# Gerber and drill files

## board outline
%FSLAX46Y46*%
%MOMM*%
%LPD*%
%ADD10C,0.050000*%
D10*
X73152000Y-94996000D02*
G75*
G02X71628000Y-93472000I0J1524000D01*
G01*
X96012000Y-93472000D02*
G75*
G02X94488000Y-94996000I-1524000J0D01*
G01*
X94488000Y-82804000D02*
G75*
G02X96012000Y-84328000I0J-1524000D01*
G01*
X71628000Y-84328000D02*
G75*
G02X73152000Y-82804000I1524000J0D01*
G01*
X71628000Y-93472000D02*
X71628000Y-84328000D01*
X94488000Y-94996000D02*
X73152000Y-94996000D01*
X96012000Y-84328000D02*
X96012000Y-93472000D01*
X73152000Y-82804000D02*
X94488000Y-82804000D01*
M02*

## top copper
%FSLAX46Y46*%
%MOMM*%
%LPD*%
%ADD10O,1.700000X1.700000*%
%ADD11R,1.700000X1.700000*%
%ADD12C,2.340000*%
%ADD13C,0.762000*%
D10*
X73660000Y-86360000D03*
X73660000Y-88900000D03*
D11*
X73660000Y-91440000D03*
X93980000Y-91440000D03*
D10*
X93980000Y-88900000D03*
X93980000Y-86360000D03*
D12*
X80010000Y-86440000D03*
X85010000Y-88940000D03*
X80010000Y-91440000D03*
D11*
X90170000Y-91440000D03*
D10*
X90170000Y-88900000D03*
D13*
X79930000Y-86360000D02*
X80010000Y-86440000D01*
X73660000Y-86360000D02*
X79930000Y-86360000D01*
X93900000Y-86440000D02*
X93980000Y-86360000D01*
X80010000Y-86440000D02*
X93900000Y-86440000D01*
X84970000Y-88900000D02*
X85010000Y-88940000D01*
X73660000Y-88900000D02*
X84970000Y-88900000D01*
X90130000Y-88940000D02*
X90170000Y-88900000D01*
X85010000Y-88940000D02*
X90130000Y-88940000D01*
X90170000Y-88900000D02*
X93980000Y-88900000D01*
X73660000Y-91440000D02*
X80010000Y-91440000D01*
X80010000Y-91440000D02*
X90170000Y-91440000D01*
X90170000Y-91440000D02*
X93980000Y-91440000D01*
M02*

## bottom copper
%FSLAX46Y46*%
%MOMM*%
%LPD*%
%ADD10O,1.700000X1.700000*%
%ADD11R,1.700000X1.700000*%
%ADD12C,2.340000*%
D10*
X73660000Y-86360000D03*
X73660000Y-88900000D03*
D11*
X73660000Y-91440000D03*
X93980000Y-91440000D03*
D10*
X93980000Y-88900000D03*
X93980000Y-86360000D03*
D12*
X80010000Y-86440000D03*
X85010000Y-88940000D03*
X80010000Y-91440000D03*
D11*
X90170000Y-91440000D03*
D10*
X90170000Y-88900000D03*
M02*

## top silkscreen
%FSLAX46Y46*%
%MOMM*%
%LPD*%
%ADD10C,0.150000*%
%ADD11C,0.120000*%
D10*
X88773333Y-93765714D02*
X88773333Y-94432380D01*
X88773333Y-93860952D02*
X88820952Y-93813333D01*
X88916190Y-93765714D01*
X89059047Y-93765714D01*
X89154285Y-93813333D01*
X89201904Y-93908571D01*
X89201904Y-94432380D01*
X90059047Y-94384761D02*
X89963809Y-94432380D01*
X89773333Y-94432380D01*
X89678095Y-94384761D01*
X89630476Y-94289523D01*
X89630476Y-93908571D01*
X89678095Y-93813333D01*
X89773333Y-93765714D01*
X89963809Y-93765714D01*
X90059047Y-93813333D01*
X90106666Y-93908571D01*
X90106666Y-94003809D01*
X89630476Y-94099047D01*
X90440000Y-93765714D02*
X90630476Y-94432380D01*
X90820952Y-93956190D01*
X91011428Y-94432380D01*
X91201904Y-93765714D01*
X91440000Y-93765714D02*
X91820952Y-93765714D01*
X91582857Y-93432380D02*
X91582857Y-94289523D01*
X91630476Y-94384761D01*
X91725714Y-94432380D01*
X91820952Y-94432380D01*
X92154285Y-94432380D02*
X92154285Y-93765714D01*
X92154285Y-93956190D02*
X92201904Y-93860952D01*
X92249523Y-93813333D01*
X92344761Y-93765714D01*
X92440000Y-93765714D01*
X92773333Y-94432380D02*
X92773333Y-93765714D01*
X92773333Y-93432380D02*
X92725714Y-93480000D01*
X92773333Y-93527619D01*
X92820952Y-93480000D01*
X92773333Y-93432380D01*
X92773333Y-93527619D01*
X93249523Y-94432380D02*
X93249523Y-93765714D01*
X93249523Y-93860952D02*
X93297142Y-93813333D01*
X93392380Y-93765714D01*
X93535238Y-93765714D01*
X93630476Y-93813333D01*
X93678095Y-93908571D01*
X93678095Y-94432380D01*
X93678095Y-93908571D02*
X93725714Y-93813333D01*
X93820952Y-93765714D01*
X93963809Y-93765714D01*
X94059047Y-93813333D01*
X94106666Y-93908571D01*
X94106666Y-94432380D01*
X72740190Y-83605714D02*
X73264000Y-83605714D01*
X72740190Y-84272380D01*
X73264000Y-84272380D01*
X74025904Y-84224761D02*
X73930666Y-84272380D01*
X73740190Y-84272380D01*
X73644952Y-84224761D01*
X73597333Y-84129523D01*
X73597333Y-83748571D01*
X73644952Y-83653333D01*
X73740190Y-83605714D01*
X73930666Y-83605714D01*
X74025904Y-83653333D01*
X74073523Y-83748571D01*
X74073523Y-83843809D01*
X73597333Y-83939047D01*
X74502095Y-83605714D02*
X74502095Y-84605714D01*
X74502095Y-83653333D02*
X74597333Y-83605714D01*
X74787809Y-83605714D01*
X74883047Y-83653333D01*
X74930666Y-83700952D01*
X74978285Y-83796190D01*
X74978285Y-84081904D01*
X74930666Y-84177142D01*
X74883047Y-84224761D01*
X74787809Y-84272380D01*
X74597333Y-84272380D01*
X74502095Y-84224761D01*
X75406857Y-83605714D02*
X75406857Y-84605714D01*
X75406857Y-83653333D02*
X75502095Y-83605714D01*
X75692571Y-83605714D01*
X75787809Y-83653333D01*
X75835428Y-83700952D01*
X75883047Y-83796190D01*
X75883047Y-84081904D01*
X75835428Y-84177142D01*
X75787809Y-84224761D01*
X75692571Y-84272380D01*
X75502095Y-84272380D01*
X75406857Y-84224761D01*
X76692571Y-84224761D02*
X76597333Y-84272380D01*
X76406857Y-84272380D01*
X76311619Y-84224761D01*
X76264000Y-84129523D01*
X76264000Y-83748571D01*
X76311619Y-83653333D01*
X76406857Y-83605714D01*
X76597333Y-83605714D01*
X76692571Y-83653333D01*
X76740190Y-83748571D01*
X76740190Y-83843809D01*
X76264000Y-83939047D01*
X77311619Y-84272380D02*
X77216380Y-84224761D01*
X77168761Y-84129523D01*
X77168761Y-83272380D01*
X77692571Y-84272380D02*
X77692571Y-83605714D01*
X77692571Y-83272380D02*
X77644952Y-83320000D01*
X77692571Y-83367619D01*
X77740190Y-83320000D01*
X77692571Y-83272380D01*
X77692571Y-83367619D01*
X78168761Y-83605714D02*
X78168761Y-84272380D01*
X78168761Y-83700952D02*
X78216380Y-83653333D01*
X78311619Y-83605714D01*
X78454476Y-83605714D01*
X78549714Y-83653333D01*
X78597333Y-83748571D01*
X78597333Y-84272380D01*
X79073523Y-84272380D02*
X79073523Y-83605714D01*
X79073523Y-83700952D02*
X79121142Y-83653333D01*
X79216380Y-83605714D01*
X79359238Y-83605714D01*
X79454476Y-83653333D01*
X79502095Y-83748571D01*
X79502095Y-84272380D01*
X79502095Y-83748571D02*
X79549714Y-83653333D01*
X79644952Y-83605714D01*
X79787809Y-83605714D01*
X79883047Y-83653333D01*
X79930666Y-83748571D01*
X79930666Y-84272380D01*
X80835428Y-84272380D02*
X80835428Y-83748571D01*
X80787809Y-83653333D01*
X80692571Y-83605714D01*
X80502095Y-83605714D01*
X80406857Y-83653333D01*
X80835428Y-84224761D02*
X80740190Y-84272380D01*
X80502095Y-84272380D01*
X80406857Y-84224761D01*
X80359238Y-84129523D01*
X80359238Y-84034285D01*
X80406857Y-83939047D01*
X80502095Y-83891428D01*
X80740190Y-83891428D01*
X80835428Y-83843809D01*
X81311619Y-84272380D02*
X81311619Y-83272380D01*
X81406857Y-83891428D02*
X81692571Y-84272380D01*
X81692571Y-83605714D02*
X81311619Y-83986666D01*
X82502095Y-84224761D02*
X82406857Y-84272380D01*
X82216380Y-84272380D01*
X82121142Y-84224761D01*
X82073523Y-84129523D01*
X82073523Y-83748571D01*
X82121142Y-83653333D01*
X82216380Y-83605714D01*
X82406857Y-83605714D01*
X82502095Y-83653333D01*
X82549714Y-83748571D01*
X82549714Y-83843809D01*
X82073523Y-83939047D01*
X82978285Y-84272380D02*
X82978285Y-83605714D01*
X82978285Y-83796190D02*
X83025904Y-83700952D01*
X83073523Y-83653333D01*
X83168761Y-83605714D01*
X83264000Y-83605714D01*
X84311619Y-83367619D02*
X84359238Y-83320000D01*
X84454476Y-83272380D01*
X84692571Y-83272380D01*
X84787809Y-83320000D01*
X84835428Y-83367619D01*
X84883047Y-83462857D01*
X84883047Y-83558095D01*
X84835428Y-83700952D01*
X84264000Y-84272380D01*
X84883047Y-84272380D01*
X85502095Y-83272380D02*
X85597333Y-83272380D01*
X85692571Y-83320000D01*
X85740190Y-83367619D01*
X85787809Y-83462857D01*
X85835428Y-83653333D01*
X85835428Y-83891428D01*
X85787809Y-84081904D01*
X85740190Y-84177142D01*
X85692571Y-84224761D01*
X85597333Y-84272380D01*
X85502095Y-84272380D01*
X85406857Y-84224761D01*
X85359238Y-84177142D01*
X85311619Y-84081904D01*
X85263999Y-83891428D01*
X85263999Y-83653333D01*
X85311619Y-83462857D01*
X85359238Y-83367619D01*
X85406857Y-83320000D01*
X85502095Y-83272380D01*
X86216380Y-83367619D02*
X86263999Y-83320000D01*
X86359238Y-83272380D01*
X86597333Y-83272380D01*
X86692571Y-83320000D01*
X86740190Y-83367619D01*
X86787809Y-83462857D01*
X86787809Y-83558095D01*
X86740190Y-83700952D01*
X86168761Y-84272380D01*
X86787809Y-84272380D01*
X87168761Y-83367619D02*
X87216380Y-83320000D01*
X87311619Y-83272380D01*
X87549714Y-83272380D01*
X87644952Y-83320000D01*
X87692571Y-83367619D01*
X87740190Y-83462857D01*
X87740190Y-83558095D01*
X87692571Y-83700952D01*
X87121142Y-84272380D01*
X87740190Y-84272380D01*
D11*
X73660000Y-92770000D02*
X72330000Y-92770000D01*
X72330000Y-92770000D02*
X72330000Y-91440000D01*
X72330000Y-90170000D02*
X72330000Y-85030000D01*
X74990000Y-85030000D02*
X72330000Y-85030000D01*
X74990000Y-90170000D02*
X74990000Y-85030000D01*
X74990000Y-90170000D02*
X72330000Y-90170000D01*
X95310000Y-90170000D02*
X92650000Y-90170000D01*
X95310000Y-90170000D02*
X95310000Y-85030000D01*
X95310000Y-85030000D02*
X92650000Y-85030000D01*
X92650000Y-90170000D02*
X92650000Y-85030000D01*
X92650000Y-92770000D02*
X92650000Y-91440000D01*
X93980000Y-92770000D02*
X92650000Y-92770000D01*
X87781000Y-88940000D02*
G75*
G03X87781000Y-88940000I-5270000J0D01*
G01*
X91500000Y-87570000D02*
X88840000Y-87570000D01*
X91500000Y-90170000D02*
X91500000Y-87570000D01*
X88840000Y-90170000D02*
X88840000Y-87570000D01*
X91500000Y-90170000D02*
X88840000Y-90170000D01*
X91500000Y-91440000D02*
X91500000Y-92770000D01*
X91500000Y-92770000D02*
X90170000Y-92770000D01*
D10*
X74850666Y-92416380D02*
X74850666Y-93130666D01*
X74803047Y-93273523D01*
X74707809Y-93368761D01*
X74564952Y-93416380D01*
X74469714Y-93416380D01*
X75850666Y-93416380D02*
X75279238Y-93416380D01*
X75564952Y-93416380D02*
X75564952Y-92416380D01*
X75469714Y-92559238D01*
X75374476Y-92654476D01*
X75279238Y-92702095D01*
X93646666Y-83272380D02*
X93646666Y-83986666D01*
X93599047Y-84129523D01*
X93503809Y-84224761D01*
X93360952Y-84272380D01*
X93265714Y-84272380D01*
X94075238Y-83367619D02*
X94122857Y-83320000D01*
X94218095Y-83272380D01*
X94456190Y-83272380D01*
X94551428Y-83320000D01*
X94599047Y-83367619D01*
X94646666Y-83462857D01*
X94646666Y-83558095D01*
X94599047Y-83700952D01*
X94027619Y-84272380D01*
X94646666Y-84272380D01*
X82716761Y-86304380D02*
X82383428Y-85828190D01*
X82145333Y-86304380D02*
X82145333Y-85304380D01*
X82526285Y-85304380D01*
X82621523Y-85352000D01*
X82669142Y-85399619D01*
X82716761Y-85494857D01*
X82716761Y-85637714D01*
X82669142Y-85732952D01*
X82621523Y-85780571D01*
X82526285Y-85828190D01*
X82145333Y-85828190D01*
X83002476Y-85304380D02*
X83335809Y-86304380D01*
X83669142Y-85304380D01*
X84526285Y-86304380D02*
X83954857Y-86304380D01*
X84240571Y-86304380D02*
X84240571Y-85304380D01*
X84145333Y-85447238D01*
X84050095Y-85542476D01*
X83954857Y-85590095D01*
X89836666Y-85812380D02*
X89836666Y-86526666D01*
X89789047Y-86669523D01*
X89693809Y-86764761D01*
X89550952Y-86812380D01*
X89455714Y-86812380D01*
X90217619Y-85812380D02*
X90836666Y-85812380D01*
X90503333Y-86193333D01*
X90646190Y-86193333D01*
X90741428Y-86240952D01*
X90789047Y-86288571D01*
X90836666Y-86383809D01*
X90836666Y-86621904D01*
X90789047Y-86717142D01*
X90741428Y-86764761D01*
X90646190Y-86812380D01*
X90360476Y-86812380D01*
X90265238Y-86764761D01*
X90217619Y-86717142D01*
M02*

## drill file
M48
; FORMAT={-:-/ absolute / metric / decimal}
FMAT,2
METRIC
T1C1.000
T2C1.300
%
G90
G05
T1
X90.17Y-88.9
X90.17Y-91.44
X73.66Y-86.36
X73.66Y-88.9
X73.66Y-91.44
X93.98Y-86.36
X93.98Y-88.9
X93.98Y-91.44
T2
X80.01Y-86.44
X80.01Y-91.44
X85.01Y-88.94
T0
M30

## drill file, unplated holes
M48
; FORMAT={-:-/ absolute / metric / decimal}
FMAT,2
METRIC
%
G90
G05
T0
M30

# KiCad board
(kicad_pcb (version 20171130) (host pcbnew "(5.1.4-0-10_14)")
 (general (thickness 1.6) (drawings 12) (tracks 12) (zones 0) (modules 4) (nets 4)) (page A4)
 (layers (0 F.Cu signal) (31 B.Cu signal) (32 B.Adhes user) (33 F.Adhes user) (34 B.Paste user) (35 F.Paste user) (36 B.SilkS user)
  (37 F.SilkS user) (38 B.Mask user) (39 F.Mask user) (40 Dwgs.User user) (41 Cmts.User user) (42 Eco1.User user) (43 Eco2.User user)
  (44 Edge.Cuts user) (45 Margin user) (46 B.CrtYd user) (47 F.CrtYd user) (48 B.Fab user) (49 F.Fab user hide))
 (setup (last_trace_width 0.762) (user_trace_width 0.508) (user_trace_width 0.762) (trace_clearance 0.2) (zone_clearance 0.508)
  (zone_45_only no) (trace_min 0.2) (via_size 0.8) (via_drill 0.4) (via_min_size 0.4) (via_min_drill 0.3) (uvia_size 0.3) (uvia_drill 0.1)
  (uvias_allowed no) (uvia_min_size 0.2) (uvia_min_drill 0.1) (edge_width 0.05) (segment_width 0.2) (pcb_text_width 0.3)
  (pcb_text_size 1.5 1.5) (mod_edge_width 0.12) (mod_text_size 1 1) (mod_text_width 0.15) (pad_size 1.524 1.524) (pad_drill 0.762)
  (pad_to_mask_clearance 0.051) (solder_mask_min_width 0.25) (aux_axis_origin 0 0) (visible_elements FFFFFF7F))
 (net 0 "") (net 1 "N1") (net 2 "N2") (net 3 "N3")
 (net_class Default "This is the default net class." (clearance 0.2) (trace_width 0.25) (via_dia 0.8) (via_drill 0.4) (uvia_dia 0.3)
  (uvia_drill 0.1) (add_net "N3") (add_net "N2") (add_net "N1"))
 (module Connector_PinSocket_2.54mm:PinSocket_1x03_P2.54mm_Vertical (layer F.Cu) (at 73.66 91.44 180)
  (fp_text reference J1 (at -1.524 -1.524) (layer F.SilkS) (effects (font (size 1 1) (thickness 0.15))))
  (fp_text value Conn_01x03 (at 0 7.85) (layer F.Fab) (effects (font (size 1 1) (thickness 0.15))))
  (fp_line (start 0 -1.33) (end 1.33 -1.33) (layer F.SilkS) (width 0.12))
  (fp_line (start 1.33 -1.33) (end 1.33 0) (layer F.SilkS) (width 0.12))
  (fp_line (start 1.33 1.27) (end 1.33 6.41) (layer F.SilkS) (width 0.12))
  (fp_line (start -1.33 6.41) (end 1.33 6.41) (layer F.SilkS) (width 0.12))
  (fp_line (start -1.33 1.27) (end -1.33 6.41) (layer F.SilkS) (width 0.12))
  (fp_line (start -1.33 1.27) (end 1.33 1.27) (layer F.SilkS) (width 0.12))
  (pad 3 thru_hole oval (at 0 5.08 180) (size 1.7 1.7) (drill 1) (layers *.Cu *.Mask) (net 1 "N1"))
  (pad 2 thru_hole oval (at 0 2.54 180) (size 1.7 1.7) (drill 1) (layers *.Cu *.Mask) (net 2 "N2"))
  (pad 1 thru_hole rect (at 0 0 180) (size 1.7 1.7) (drill 1) (layers *.Cu *.Mask) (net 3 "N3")))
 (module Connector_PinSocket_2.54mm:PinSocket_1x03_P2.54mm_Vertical (layer F.Cu) (at 93.98 91.44 180)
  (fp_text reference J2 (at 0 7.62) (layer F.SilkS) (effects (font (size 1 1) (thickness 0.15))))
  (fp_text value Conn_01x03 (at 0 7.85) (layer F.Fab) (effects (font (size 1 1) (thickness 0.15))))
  (fp_line (start -1.33 1.27) (end 1.33 1.27) (layer F.SilkS) (width 0.12))
  (fp_line (start -1.33 1.27) (end -1.33 6.41) (layer F.SilkS) (width 0.12))
  (fp_line (start -1.33 6.41) (end 1.33 6.41) (layer F.SilkS) (width 0.12))
  (fp_line (start 1.33 1.27) (end 1.33 6.41) (layer F.SilkS) (width 0.12))
  (fp_line (start 1.33 -1.33) (end 1.33 0) (layer F.SilkS) (width 0.12))
  (fp_line (start 0 -1.33) (end 1.33 -1.33) (layer F.SilkS) (width 0.12))
  (pad 1 thru_hole rect (at 0 0 180) (size 1.7 1.7) (drill 1) (layers *.Cu *.Mask) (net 3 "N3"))
  (pad 2 thru_hole oval (at 0 2.54 180) (size 1.7 1.7) (drill 1) (layers *.Cu *.Mask) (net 2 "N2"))
  (pad 3 thru_hole oval (at 0 5.08 180) (size 1.7 1.7) (drill 1) (layers *.Cu *.Mask) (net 1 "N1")))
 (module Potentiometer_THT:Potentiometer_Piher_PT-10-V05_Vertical (layer F.Cu) (at 80.01 91.44)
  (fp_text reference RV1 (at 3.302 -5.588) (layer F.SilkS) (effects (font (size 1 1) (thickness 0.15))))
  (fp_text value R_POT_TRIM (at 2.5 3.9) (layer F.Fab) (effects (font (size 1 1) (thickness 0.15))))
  (fp_circle (center 2.501 -2.5) (end 7.771 -2.5) (layer F.SilkS) (width 0.12))
  (pad 3 thru_hole circle (at 0 -5) (size 2.34 2.34) (drill 1.3) (layers *.Cu *.Mask) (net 1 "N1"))
  (pad 2 thru_hole circle (at 5 -2.5) (size 2.34 2.34) (drill 1.3) (layers *.Cu *.Mask) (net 2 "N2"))
  (pad 1 thru_hole circle (at 0 0) (size 2.34 2.34) (drill 1.3) (layers *.Cu *.Mask) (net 3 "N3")))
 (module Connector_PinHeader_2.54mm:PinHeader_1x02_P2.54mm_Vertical (layer F.Cu) (at 90.17 91.44 180)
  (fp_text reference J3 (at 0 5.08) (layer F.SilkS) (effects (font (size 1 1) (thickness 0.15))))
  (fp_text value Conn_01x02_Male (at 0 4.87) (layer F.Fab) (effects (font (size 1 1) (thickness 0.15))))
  (fp_line (start -1.33 3.87) (end 1.33 3.87) (layer F.SilkS) (width 0.12))
  (fp_line (start -1.33 1.27) (end -1.33 3.87) (layer F.SilkS) (width 0.12))
  (fp_line (start 1.33 1.27) (end 1.33 3.87) (layer F.SilkS) (width 0.12))
  (fp_line (start -1.33 1.27) (end 1.33 1.27) (layer F.SilkS) (width 0.12))
  (fp_line (start -1.33 0) (end -1.33 -1.33) (layer F.SilkS) (width 0.12))
  (fp_line (start -1.33 -1.33) (end 0 -1.33) (layer F.SilkS) (width 0.12))
  (pad 1 thru_hole rect (at 0 0 180) (size 1.7 1.7) (drill 1) (layers *.Cu *.Mask) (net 3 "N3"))
  (pad 2 thru_hole oval (at 0 2.54 180) (size 1.7 1.7) (drill 1) (layers *.Cu *.Mask) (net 2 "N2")))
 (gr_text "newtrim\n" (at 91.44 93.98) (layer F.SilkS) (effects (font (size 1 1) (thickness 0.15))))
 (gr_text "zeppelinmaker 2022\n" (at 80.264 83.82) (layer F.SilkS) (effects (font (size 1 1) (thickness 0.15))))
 (gr_arc (start 73.152 93.472) (end 71.628 93.472) (angle -90) (layer Edge.Cuts) (width 0.05))
 (gr_arc (start 94.488 93.472) (end 94.488 94.996) (angle -90) (layer Edge.Cuts) (width 0.05))
 (gr_arc (start 94.488 84.328) (end 96.012 84.328) (angle -90) (layer Edge.Cuts) (width 0.05))
 (gr_arc (start 73.152 84.328) (end 73.152 82.804) (angle -90) (layer Edge.Cuts) (width 0.05))
 (gr_line (start 71.628 93.472) (end 71.628 84.328) (layer Edge.Cuts) (width 0.05))
 (gr_line (start 94.488 94.996) (end 73.152 94.996) (layer Edge.Cuts) (width 0.05))
 (gr_line (start 96.012 84.328) (end 96.012 93.472) (layer Edge.Cuts) (width 0.05))
 (gr_line (start 73.152 82.804) (end 94.488 82.804) (layer Edge.Cuts) (width 0.05))
 (segment (start 79.93 86.36) (end 80.01 86.44) (width 0.762) (layer F.Cu) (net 1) (status 30))
 (segment (start 73.66 86.36) (end 79.93 86.36) (width 0.762) (layer F.Cu) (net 1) (status 30))
 (segment (start 93.9 86.44) (end 93.98 86.36) (width 0.762) (layer F.Cu) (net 1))
 (segment (start 80.01 86.44) (end 93.9 86.44) (width 0.762) (layer F.Cu) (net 1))
 (segment (start 84.97 88.9) (end 85.01 88.94) (width 0.762) (layer F.Cu) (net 2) (status 30))
 (segment (start 73.66 88.9) (end 84.97 88.9) (width 0.762) (layer F.Cu) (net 2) (status 30))
 (segment (start 90.13 88.94) (end 90.17 88.9) (width 0.762) (layer F.Cu) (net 2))
 (segment (start 85.01 88.94) (end 90.13 88.94) (width 0.762) (layer F.Cu) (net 2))
 (segment (start 90.17 88.9) (end 93.98 88.9) (width 0.762) (layer F.Cu) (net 2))
 (segment (start 73.66 91.44) (end 80.01 91.44) (width 0.762) (layer F.Cu) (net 3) (status 30))
 (segment (start 80.01 91.44) (end 90.17 91.44) (width 0.762) (layer F.Cu) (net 3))
 (segment (start 90.17 91.44) (end 93.98 91.44) (width 0.762) (layer F.Cu) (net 3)))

